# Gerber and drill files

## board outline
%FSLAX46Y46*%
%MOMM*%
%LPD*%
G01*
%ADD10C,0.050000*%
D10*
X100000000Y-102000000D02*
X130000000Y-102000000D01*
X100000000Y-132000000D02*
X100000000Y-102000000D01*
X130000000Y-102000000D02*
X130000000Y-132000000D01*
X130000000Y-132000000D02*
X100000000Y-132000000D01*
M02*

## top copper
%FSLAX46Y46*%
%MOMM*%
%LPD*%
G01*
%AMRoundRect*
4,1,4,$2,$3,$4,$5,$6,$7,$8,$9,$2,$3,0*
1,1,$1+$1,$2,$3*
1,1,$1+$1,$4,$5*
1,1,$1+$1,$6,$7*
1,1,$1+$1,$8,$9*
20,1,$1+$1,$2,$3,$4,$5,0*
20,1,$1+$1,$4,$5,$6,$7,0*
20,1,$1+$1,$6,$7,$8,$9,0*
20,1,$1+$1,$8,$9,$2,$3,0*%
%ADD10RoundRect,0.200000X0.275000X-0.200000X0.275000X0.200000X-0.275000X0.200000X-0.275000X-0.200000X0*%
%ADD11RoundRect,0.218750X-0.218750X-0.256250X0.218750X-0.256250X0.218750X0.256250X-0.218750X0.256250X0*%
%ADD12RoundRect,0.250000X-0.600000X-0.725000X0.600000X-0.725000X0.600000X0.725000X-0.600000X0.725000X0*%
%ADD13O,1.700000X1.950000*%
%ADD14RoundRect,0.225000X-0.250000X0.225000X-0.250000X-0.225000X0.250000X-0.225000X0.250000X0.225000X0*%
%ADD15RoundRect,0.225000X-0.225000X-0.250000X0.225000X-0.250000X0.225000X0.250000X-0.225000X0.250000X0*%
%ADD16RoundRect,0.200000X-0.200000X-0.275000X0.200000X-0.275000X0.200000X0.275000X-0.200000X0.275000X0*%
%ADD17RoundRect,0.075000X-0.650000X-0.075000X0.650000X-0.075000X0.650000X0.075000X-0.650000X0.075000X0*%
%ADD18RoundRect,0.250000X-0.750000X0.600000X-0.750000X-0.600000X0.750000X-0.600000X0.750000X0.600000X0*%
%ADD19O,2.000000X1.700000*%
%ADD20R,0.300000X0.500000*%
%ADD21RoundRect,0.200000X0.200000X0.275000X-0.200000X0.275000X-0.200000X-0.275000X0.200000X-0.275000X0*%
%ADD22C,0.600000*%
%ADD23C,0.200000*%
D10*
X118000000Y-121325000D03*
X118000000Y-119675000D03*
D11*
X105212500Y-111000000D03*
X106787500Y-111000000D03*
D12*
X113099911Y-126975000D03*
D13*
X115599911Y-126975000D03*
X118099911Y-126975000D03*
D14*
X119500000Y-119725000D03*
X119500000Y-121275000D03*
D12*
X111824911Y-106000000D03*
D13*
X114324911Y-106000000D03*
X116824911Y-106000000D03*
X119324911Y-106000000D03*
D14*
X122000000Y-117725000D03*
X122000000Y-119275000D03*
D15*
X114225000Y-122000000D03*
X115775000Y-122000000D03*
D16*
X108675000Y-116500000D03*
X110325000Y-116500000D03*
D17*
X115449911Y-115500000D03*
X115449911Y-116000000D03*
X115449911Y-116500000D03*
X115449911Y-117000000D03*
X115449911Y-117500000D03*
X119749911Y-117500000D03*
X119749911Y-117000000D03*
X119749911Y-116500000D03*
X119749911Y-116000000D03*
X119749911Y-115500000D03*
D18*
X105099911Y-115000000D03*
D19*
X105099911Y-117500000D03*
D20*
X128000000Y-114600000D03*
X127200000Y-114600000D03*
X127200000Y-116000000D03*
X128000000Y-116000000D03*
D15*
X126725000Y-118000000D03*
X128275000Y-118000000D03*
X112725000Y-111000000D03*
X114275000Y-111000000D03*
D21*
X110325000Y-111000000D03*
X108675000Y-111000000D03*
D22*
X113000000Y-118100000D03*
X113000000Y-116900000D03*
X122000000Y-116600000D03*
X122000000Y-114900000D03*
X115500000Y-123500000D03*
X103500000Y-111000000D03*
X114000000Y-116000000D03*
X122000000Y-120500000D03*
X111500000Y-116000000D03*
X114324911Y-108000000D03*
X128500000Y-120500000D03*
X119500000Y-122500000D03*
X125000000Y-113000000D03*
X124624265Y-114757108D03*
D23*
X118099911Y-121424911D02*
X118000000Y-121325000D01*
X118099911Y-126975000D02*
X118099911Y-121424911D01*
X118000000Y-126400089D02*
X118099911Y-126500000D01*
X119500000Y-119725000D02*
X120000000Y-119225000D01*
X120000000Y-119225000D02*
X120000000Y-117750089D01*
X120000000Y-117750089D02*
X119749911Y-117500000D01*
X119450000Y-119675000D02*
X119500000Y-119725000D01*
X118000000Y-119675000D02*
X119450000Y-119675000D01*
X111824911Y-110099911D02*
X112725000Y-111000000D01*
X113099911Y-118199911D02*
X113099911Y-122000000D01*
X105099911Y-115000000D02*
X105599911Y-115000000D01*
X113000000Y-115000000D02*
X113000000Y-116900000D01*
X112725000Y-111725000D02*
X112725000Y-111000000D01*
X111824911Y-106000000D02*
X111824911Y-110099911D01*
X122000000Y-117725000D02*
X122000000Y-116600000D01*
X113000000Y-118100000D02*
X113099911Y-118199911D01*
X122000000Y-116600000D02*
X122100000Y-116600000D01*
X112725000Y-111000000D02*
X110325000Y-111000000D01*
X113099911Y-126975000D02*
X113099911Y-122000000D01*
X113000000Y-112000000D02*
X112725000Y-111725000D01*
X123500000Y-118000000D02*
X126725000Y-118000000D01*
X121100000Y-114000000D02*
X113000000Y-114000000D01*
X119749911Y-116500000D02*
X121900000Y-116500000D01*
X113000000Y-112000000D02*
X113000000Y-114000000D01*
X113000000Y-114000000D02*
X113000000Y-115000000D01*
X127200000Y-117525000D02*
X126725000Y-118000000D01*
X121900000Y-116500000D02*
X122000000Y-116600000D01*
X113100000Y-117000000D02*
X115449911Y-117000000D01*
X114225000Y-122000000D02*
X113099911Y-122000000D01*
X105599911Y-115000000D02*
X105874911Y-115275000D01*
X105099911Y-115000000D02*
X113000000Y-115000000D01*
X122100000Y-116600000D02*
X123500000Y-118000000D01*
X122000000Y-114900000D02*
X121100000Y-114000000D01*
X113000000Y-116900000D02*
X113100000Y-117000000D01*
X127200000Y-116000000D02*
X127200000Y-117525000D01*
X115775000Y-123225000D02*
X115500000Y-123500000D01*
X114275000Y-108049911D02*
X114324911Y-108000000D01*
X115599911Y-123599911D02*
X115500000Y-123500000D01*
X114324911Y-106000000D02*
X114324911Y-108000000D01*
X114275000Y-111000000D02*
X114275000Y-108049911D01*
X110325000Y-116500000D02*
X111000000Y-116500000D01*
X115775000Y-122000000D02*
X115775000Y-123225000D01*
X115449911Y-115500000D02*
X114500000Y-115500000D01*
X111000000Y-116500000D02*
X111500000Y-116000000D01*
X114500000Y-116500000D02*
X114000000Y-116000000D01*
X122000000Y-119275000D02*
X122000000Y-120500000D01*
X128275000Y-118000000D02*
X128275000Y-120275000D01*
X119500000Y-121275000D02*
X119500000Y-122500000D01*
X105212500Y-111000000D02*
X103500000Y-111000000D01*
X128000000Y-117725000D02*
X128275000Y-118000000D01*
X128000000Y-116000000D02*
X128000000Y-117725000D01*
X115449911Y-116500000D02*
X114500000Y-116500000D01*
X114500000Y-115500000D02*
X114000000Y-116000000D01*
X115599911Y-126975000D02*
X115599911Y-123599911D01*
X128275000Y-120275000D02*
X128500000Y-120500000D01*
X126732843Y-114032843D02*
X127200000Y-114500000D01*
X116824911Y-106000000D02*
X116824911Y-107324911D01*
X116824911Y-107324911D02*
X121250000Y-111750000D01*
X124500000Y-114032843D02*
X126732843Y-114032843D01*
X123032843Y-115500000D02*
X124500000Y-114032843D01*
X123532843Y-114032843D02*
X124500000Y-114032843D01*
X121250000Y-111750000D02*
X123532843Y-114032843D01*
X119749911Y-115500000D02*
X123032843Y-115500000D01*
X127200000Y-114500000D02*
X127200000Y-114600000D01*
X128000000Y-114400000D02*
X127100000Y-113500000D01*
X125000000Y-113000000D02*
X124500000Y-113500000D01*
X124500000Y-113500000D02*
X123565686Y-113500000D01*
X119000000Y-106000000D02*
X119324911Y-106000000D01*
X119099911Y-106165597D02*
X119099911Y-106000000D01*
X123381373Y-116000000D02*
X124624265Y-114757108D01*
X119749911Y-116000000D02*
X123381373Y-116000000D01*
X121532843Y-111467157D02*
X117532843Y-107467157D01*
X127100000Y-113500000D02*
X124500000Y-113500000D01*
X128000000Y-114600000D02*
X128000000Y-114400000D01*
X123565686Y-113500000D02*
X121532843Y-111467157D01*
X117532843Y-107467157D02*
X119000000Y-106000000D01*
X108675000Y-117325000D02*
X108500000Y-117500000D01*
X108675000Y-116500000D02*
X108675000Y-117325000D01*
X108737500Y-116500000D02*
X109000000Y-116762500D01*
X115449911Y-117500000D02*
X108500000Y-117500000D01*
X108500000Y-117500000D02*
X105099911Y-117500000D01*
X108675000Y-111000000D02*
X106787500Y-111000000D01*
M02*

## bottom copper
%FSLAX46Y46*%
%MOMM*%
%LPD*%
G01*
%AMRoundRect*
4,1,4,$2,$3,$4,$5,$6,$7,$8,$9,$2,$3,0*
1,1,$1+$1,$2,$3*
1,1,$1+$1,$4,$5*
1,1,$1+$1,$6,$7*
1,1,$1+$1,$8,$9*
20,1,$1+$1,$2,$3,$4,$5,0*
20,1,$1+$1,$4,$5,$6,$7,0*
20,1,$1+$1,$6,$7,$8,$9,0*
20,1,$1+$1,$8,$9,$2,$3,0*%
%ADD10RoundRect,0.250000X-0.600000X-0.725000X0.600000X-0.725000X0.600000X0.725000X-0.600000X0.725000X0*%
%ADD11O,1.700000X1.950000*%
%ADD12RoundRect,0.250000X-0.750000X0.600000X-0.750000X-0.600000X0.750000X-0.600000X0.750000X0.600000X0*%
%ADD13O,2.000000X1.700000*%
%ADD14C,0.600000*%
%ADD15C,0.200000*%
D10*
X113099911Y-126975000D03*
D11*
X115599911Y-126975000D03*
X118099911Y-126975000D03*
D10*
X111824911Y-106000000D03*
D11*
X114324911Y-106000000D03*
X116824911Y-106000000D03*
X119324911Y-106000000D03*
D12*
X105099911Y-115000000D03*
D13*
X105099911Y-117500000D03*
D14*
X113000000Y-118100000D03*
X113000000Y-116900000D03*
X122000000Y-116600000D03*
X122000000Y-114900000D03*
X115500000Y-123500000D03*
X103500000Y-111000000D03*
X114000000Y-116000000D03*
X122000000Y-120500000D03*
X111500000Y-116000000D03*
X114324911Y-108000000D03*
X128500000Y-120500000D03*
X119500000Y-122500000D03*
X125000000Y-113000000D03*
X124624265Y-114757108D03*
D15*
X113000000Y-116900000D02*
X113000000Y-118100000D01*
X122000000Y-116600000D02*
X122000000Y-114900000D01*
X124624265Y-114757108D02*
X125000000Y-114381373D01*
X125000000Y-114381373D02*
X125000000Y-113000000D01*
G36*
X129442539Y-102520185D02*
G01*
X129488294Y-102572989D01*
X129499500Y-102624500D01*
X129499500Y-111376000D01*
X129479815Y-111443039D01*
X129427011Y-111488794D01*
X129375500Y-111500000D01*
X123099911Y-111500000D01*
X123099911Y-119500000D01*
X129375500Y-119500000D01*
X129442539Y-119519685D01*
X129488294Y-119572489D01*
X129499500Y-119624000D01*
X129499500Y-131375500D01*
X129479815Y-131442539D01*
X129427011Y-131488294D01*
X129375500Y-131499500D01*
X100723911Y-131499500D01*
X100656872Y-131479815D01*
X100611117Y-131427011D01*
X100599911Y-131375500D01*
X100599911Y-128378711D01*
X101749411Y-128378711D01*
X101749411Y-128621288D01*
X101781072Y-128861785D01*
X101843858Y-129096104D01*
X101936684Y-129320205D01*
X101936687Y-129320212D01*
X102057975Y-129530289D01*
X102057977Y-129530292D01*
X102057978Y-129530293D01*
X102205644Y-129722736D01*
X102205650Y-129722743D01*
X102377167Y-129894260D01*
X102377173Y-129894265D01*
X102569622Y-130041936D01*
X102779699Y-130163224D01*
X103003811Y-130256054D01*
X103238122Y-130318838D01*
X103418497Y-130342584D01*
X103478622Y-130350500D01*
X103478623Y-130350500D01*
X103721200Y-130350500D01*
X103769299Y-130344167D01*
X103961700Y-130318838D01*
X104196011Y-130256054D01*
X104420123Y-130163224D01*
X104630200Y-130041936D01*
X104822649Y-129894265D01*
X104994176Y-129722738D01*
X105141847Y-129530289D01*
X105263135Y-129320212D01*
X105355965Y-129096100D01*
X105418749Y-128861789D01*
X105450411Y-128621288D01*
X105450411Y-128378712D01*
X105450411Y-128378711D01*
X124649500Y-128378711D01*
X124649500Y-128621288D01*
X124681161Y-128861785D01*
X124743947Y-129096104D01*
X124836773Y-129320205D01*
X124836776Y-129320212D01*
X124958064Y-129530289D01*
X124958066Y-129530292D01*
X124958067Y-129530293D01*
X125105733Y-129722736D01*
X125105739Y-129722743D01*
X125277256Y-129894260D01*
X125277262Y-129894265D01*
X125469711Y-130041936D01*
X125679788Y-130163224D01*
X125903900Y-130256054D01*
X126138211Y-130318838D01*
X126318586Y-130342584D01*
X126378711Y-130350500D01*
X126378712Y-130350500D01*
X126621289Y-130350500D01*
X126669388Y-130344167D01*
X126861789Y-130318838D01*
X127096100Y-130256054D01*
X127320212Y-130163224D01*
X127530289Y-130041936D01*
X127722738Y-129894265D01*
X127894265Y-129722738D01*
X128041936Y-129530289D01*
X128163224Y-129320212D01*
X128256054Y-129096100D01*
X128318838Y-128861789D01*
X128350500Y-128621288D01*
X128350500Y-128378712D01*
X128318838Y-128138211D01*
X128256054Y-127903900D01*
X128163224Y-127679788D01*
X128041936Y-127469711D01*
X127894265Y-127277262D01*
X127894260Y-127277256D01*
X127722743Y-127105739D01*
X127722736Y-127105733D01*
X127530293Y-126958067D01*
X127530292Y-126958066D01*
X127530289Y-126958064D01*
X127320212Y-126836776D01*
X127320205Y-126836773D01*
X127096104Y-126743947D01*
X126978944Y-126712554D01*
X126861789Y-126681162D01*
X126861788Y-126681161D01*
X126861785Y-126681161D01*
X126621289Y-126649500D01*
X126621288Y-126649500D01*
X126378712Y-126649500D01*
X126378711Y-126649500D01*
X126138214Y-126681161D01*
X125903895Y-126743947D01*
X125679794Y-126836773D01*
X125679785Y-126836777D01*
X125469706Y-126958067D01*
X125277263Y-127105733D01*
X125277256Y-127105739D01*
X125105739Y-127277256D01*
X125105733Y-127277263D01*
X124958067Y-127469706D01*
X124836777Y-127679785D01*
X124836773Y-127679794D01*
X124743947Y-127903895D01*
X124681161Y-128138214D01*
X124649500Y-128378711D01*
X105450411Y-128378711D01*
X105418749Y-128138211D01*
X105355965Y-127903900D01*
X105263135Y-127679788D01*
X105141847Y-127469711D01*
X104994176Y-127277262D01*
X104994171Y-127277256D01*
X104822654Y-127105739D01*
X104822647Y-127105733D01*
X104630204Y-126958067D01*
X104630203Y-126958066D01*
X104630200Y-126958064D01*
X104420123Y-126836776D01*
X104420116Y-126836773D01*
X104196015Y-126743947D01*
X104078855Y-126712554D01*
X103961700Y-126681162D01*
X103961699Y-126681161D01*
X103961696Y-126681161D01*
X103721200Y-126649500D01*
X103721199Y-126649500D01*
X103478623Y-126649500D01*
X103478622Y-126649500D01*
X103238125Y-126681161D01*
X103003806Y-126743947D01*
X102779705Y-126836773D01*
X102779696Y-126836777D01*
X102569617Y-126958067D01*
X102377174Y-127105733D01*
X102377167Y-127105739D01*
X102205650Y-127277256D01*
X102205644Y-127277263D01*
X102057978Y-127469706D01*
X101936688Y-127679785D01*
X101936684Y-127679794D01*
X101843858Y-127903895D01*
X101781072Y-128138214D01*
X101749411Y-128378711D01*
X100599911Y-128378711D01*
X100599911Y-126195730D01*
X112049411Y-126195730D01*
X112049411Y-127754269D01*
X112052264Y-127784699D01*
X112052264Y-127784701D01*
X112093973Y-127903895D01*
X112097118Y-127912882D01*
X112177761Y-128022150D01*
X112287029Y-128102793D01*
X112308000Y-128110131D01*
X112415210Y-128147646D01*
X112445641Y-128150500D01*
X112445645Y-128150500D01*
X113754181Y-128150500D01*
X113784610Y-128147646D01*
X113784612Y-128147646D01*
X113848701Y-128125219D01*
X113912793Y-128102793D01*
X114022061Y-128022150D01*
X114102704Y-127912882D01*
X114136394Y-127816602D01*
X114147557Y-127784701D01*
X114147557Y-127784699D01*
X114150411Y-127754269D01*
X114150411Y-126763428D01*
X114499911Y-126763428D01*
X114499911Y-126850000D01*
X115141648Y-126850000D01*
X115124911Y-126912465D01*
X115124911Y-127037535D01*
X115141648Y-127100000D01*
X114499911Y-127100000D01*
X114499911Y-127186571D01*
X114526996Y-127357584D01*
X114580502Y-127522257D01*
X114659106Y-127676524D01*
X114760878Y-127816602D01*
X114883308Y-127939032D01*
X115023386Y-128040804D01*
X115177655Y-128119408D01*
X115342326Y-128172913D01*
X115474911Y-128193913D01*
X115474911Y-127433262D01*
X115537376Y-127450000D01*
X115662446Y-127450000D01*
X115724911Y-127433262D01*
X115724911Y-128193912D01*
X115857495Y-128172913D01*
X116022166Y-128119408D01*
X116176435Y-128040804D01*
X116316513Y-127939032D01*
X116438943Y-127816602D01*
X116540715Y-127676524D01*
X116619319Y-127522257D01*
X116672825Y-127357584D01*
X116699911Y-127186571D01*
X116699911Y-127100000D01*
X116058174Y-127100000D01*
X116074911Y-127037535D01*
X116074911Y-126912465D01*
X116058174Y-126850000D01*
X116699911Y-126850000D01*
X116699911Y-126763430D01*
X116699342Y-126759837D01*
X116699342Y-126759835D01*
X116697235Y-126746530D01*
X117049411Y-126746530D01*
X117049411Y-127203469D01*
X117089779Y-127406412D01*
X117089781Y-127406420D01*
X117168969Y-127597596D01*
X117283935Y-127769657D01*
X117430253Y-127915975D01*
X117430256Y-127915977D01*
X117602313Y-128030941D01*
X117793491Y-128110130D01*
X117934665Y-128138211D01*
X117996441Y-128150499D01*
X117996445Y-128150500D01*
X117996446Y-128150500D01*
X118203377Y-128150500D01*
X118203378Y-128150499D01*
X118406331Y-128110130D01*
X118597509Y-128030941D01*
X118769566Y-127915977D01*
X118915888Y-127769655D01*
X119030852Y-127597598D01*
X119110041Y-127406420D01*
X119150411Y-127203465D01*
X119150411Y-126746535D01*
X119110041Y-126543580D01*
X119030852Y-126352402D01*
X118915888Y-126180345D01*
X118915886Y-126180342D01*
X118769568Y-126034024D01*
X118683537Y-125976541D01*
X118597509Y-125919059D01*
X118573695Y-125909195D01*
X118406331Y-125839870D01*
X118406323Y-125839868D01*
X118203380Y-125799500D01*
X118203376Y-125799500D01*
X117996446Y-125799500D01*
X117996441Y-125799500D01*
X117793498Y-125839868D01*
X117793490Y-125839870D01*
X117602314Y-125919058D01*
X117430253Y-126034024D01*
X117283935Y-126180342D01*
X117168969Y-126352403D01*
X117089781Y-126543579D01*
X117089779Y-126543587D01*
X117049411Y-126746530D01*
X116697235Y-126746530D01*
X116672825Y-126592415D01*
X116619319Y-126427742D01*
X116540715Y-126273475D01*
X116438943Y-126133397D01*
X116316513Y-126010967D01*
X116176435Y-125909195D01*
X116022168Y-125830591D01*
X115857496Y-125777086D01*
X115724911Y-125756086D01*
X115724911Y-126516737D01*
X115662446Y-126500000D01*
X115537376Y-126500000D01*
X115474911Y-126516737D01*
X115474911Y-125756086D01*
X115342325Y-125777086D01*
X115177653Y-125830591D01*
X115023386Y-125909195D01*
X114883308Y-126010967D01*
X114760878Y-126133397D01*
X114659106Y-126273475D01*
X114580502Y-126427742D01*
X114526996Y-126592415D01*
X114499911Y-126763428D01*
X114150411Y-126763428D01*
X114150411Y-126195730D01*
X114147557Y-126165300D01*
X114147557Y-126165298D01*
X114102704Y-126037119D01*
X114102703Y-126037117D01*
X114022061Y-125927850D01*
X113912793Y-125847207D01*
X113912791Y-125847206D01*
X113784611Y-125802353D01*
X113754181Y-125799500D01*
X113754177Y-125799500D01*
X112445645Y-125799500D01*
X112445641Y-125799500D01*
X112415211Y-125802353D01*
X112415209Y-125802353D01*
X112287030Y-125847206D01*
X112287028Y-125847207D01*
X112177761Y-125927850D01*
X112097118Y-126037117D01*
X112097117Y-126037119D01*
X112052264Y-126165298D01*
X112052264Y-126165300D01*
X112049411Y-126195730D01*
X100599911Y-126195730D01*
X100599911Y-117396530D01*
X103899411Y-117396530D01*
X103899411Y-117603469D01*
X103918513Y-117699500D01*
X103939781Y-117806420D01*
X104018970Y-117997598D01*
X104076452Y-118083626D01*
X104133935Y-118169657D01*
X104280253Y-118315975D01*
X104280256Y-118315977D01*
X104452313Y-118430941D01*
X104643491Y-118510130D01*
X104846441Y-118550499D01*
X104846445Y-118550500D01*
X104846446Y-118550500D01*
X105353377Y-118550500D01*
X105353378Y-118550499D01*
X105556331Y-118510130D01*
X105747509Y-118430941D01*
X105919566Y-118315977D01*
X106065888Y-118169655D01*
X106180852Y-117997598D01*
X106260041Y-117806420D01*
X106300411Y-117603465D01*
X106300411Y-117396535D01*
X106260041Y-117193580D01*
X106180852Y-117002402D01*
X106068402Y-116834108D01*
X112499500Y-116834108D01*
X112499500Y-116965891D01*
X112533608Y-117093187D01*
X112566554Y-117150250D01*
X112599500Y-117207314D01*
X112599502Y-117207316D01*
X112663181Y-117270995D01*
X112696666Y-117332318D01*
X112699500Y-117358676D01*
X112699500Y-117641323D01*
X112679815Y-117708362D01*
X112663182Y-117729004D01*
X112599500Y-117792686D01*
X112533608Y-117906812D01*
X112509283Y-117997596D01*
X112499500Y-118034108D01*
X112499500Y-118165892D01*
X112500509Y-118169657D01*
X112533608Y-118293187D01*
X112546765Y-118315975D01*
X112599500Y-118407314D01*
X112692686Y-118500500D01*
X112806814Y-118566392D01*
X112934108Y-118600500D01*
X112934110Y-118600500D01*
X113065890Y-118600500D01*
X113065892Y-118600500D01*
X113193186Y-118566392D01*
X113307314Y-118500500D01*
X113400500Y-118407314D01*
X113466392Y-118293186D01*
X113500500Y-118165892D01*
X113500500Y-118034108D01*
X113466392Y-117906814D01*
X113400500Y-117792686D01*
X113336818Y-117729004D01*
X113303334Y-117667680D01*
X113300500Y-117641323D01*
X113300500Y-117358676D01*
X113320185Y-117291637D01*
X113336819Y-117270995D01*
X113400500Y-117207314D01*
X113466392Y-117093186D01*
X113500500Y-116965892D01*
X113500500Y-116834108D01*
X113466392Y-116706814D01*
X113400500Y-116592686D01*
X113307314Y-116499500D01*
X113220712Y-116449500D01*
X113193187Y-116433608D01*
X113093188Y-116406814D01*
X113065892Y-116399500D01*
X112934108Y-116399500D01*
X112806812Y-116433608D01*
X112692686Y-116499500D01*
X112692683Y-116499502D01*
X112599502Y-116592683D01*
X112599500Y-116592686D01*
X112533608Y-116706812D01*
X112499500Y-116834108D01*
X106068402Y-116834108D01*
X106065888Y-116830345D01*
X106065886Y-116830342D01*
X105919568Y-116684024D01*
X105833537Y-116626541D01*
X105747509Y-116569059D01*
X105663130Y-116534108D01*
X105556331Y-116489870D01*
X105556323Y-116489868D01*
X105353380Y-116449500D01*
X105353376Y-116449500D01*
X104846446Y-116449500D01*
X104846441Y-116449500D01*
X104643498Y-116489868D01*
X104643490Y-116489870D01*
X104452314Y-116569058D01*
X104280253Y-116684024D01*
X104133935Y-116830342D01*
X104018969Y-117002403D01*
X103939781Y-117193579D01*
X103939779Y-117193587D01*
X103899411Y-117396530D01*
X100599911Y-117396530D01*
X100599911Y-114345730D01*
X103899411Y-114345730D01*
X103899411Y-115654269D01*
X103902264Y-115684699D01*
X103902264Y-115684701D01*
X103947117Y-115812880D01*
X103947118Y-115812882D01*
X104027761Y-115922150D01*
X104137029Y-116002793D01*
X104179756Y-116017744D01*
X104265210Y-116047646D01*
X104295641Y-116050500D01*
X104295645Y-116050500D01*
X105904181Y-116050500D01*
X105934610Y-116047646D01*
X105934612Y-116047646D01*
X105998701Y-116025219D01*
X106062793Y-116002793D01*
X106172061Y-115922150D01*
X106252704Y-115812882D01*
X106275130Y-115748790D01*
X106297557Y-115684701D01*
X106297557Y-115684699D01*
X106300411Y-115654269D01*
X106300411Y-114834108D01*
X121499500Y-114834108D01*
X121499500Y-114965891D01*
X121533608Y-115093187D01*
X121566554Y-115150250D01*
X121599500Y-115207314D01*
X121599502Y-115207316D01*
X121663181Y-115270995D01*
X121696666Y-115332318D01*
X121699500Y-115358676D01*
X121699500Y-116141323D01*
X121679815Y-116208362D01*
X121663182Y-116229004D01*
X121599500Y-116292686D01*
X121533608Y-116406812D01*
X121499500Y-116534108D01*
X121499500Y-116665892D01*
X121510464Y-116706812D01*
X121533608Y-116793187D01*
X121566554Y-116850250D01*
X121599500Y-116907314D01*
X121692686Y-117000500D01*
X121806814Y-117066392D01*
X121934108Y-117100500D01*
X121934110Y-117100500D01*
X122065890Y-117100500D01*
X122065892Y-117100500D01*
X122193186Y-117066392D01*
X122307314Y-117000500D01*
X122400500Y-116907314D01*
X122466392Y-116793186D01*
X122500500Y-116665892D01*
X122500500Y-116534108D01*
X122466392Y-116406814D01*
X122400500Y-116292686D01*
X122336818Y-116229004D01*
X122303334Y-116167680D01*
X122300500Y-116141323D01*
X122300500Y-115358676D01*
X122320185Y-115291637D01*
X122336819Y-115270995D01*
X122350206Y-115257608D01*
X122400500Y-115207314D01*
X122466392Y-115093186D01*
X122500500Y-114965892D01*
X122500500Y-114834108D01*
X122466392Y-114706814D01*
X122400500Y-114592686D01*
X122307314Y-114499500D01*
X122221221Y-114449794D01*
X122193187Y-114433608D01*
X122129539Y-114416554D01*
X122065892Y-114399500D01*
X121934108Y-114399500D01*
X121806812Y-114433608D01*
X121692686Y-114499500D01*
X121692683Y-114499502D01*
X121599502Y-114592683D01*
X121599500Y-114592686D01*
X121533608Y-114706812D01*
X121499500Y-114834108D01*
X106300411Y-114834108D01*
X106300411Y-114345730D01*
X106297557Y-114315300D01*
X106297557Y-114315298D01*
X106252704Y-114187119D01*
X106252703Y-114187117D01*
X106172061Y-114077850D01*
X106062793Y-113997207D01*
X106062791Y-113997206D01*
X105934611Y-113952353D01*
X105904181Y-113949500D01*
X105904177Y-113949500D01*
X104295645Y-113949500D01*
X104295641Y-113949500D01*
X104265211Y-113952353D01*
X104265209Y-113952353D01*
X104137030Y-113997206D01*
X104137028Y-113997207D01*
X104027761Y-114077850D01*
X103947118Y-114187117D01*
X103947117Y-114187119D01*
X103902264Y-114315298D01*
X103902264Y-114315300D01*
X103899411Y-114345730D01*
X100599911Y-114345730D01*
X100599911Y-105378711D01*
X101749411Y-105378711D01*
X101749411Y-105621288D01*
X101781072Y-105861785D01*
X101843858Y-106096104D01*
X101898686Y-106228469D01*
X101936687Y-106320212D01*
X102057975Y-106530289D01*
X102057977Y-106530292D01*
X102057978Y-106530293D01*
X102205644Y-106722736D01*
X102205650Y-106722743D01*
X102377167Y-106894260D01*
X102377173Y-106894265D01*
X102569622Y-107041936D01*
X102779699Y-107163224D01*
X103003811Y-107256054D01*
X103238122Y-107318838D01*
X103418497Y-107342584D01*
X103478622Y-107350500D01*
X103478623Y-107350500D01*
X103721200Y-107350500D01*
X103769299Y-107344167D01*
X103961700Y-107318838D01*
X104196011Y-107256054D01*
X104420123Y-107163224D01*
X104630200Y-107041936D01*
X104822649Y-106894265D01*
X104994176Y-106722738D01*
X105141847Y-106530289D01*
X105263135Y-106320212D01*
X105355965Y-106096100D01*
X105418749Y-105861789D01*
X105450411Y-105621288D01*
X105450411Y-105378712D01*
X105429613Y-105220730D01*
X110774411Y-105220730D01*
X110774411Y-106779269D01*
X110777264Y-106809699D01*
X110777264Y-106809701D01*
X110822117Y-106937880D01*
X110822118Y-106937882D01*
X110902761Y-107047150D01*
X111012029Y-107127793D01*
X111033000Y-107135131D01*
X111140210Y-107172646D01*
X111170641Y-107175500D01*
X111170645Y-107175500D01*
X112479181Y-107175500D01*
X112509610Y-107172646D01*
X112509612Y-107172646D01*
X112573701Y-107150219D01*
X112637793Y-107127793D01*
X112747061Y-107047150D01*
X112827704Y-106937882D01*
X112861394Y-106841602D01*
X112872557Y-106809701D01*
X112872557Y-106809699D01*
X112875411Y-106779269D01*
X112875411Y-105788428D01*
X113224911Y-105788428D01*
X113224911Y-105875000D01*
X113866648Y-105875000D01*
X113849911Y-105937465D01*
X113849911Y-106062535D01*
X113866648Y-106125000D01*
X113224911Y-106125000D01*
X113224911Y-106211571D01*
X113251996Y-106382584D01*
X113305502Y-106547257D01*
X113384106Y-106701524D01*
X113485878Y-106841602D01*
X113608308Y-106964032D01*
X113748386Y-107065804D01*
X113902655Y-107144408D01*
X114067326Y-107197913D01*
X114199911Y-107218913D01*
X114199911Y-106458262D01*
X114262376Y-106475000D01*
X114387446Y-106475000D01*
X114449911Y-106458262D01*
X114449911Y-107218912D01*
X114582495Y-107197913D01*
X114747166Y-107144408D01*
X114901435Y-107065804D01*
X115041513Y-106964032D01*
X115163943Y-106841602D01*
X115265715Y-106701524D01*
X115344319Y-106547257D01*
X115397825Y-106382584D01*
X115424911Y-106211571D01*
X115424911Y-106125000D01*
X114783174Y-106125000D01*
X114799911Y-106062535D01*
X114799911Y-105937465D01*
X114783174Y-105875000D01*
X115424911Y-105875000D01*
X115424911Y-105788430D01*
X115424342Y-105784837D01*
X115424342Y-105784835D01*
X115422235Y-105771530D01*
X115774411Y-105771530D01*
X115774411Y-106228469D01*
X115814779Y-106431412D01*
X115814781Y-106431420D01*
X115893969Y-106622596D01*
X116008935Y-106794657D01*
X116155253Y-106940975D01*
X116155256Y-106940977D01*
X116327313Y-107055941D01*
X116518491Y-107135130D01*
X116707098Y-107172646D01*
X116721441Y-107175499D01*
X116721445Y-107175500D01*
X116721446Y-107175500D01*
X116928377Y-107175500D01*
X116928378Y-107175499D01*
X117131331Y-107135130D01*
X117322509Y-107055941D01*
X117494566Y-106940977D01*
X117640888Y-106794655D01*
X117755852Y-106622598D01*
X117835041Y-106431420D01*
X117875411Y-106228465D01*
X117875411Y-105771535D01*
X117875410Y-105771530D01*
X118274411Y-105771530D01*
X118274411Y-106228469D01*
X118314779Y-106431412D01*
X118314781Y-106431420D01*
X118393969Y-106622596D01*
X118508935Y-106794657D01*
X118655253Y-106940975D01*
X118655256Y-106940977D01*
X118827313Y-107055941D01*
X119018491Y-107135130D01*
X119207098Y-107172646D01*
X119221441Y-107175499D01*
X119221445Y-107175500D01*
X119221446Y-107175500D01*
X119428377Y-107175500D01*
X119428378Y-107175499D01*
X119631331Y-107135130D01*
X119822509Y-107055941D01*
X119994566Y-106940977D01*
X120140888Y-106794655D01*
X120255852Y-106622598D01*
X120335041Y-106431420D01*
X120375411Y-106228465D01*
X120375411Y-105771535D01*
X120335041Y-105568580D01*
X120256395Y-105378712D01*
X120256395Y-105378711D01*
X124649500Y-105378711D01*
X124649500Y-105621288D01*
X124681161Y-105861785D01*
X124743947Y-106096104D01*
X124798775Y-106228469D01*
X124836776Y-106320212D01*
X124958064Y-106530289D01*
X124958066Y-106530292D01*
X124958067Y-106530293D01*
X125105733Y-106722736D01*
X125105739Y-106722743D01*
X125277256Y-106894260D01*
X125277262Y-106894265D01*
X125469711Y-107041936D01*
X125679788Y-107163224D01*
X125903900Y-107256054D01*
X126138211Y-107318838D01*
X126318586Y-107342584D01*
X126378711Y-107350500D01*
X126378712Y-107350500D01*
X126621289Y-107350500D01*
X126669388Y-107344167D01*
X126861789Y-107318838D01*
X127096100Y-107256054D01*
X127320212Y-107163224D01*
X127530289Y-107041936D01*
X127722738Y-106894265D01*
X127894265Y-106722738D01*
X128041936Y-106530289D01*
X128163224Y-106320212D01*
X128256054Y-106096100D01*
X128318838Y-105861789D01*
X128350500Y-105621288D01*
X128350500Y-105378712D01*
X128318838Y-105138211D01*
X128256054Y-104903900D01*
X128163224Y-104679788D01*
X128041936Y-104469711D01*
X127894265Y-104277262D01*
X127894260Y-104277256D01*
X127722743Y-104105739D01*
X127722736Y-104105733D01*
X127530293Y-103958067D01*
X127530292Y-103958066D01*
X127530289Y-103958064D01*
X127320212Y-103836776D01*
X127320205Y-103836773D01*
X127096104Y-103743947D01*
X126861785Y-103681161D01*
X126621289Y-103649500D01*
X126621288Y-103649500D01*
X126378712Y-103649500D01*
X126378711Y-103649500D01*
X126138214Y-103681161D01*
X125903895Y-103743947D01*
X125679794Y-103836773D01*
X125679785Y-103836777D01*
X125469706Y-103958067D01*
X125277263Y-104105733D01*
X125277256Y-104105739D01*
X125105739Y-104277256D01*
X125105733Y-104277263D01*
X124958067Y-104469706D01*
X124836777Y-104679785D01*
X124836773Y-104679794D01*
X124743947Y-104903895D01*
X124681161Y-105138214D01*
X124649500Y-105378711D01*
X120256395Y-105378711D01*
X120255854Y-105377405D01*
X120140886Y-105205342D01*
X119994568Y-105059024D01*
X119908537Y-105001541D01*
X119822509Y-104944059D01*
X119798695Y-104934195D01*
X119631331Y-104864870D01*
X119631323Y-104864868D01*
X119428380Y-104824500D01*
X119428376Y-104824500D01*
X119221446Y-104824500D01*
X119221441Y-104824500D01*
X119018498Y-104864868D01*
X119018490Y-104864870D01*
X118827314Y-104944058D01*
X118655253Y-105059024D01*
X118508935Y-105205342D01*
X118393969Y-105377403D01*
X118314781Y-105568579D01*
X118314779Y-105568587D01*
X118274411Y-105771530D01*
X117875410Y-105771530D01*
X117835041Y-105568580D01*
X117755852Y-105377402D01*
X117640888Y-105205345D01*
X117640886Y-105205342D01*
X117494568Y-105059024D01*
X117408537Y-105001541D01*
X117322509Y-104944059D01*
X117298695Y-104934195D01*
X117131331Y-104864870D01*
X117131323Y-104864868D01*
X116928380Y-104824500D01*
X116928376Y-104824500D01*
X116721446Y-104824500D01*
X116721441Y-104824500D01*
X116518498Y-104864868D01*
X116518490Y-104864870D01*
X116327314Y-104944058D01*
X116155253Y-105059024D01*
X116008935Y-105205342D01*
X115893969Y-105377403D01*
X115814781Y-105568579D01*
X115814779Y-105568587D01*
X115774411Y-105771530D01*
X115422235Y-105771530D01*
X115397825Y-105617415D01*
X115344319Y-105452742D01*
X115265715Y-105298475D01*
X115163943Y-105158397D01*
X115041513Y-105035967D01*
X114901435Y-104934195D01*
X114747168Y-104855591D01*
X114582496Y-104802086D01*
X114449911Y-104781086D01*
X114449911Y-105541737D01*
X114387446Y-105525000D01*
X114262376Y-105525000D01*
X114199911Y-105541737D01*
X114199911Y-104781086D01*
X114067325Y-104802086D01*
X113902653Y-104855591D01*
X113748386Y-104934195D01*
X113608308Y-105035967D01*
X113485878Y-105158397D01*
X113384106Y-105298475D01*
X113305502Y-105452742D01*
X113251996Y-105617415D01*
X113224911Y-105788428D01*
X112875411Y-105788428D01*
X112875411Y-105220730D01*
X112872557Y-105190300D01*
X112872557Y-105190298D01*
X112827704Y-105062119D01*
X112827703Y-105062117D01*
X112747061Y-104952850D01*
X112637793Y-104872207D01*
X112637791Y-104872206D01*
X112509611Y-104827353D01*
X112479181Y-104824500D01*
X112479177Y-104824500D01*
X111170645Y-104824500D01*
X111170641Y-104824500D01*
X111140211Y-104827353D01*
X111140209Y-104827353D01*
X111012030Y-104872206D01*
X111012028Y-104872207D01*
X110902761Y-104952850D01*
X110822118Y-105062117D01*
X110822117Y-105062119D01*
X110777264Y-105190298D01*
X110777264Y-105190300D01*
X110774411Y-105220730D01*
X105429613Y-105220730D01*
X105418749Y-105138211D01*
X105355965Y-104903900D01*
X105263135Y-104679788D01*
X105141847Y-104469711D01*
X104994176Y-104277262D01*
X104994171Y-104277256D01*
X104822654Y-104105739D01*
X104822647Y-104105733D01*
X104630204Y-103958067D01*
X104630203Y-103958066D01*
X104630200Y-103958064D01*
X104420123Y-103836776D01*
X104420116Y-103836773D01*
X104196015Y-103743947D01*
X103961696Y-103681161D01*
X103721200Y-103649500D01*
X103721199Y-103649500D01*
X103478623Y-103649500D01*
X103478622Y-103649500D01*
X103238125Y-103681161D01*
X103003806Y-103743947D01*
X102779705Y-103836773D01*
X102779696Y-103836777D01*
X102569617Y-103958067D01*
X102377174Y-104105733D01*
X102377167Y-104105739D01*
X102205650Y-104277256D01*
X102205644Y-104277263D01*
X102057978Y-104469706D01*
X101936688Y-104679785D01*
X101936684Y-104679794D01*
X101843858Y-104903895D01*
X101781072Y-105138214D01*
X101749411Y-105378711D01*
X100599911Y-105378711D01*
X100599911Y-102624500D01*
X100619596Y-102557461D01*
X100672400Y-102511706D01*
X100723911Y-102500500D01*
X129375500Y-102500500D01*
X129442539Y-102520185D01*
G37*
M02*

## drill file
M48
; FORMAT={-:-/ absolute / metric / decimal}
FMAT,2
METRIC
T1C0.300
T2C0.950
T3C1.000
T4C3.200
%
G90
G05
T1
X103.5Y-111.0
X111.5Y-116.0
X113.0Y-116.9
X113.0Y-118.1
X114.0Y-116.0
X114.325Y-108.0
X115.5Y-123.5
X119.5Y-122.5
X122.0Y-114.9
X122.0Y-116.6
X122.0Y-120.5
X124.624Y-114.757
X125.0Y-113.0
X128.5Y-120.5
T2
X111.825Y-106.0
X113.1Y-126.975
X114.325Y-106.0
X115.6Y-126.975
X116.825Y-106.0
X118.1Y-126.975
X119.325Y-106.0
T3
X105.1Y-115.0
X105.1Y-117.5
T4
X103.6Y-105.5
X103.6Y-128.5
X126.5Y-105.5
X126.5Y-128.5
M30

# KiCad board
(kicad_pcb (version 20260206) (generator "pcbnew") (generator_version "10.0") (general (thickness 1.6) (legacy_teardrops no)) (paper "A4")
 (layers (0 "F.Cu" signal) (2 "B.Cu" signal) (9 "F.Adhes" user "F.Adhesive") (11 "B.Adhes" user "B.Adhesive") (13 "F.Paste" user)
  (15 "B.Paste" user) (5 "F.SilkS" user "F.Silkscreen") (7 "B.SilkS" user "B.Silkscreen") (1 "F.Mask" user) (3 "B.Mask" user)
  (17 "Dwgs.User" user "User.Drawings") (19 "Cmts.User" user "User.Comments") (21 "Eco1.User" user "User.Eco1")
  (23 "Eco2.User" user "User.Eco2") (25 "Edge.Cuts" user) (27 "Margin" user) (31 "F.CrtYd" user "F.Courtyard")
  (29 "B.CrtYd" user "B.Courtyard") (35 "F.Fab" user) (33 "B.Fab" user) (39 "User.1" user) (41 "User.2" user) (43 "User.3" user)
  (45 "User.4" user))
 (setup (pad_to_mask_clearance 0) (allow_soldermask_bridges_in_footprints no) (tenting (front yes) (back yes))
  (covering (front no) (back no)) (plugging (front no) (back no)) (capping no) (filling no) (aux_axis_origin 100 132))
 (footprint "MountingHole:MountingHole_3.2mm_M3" (layer "F.Cu") (at 126.5 105.5)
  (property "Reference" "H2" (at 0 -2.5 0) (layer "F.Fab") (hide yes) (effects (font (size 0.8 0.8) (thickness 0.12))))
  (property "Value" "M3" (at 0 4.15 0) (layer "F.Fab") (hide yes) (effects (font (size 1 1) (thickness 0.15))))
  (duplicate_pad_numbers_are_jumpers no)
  (pad "" np_thru_hole circle (at 0 0) (size 3.2 3.2) (drill 3.2) (layers "*.Cu" "*.Mask")))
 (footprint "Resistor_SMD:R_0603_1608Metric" (layer "F.Cu") (at 118 120.5 90)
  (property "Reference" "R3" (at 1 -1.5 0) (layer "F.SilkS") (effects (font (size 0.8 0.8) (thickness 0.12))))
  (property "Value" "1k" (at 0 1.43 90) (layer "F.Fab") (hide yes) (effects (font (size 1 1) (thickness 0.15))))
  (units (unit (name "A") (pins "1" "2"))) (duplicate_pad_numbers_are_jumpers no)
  (pad "1" smd roundrect (at -0.825 0 90) (size 0.8 0.95) (layers "F.Cu" "F.Mask" "F.Paste") (roundrect_rratio 0.25) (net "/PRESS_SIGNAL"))
  (pad "2" smd roundrect (at 0.825 0 90) (size 0.8 0.95) (layers "F.Cu" "F.Mask" "F.Paste") (roundrect_rratio 0.25) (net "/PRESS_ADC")))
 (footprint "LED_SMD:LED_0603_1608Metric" (layer "F.Cu") (at 106 111)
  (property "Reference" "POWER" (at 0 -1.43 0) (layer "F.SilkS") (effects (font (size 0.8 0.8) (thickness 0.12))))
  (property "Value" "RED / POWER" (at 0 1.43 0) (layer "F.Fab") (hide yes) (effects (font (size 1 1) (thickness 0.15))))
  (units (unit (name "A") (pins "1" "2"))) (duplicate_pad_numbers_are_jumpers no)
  (pad "1" smd roundrect (at -0.7875 0) (size 0.875 0.95) (layers "F.Cu" "F.Mask" "F.Paste") (roundrect_rratio 0.25) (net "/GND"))
  (pad "2" smd roundrect (at 0.7875 0) (size 0.875 0.95) (layers "F.Cu" "F.Mask" "F.Paste") (roundrect_rratio 0.25) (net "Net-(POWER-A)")))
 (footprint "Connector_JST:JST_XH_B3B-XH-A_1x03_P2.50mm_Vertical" (layer "F.Cu") (at 113.099911 126.975)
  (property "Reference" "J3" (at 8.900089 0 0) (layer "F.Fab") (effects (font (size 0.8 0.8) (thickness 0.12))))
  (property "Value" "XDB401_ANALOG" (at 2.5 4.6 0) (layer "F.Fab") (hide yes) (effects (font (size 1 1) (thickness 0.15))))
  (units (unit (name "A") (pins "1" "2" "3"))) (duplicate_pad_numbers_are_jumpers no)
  (pad "1" thru_hole roundrect (at 0 0) (size 1.7 1.95) (drill 0.95) (layers "*.Cu" "*.Mask") (remove_unused_layers no)
   (roundrect_rratio 0.147059) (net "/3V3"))
  (pad "2" thru_hole oval (at 2.5 0) (size 1.7 1.95) (drill 0.95) (layers "*.Cu" "*.Mask") (remove_unused_layers no) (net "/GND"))
  (pad "3" thru_hole oval (at 5 0) (size 1.7 1.95) (drill 0.95) (layers "*.Cu" "*.Mask") (remove_unused_layers no) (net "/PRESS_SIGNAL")))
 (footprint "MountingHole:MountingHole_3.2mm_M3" (layer "F.Cu") (at 126.5 128.5)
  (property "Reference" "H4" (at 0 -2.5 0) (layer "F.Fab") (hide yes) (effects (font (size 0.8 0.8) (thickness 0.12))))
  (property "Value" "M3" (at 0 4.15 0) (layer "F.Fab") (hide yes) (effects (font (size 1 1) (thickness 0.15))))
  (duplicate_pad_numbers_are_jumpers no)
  (pad "" np_thru_hole circle (at 0 0) (size 3.2 3.2) (drill 3.2) (layers "*.Cu" "*.Mask")))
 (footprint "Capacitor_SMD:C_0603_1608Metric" (layer "F.Cu") (at 119.5 120.5 -90)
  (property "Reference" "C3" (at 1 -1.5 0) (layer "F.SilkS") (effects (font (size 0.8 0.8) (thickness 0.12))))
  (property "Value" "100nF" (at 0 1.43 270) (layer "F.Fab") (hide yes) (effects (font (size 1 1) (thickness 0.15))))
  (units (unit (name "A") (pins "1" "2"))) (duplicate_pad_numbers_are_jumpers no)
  (pad "1" smd roundrect (at -0.775 0 270) (size 0.9 0.95) (layers "F.Cu" "F.Mask" "F.Paste") (roundrect_rratio 0.25) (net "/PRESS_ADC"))
  (pad "2" smd roundrect (at 0.775 0 270) (size 0.9 0.95) (layers "F.Cu" "F.Mask" "F.Paste") (roundrect_rratio 0.25) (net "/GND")))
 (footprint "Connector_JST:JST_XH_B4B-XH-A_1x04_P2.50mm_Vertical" (layer "F.Cu") (at 111.824911 106)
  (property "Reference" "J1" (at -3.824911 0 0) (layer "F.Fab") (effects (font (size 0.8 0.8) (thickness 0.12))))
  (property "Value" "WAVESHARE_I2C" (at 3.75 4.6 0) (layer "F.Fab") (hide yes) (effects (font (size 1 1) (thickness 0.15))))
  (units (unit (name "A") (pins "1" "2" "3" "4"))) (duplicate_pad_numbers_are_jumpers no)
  (pad "1" thru_hole roundrect (at 0 0) (size 1.7 1.95) (drill 0.95) (layers "*.Cu" "*.Mask") (remove_unused_layers no)
   (roundrect_rratio 0.147059) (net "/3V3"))
  (pad "2" thru_hole oval (at 2.5 0) (size 1.7 1.95) (drill 0.95) (layers "*.Cu" "*.Mask") (remove_unused_layers no) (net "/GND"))
  (pad "3" thru_hole oval (at 5 0) (size 1.7 1.95) (drill 0.95) (layers "*.Cu" "*.Mask") (remove_unused_layers no) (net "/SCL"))
  (pad "4" thru_hole oval (at 7.5 0) (size 1.7 1.95) (drill 0.95) (layers "*.Cu" "*.Mask") (remove_unused_layers no) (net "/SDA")))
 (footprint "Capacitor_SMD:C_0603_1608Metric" (layer "F.Cu") (at 122 118.5 -90)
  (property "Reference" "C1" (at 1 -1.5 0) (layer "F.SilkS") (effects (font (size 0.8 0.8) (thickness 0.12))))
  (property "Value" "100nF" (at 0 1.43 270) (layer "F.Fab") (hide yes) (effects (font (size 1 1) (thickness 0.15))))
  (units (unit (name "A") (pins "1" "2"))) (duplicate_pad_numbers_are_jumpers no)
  (pad "1" smd roundrect (at -0.775 0 270) (size 0.9 0.95) (layers "F.Cu" "F.Mask" "F.Paste") (roundrect_rratio 0.25) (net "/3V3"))
  (pad "2" smd roundrect (at 0.775 0 270) (size 0.9 0.95) (layers "F.Cu" "F.Mask" "F.Paste") (roundrect_rratio 0.25) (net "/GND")))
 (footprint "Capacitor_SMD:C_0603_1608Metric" (layer "F.Cu") (at 115 122)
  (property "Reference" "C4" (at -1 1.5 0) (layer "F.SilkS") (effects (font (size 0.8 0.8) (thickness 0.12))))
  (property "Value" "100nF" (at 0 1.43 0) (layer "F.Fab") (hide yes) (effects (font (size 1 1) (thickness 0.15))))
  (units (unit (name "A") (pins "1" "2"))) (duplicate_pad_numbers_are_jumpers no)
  (pad "1" smd roundrect (at -0.775 0) (size 0.9 0.95) (layers "F.Cu" "F.Mask" "F.Paste") (roundrect_rratio 0.25) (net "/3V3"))
  (pad "2" smd roundrect (at 0.775 0) (size 0.9 0.95) (layers "F.Cu" "F.Mask" "F.Paste") (roundrect_rratio 0.25) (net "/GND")))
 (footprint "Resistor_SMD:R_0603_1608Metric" (layer "F.Cu") (at 109.5 116.5)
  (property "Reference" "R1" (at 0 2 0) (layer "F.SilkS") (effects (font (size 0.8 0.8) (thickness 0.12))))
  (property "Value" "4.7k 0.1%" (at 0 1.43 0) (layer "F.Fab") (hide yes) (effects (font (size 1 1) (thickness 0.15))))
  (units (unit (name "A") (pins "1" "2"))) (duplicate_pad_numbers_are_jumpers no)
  (pad "1" smd roundrect (at -0.825 0) (size 0.8 0.95) (layers "F.Cu" "F.Mask" "F.Paste") (roundrect_rratio 0.25) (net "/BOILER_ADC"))
  (pad "2" smd roundrect (at 0.825 0) (size 0.8 0.95) (layers "F.Cu" "F.Mask" "F.Paste") (roundrect_rratio 0.25) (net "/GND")))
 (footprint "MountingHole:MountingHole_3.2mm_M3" (layer "F.Cu") (at 103.599911 128.5)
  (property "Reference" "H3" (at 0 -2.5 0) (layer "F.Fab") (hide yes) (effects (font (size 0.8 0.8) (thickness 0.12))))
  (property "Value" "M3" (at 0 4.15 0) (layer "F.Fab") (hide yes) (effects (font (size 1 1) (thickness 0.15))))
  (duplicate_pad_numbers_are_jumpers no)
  (pad "" np_thru_hole circle (at 0 0) (size 3.2 3.2) (drill 3.2) (layers "*.Cu" "*.Mask")))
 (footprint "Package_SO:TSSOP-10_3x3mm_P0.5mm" (layer "F.Cu") (at 117.599911 116.5)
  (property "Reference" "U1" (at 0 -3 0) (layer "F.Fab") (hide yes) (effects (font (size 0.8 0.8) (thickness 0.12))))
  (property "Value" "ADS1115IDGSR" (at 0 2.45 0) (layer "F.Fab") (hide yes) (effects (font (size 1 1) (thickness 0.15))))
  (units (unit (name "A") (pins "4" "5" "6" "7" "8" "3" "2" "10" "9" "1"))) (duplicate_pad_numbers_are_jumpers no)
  (pad "1" smd roundrect (at -2.15 -1) (size 1.45 0.3) (layers "F.Cu" "F.Mask" "F.Paste") (roundrect_rratio 0.25) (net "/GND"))
  (pad "2" smd roundrect (at -2.15 -0.5) (size 1.45 0.3) (layers "F.Cu" "F.Mask" "F.Paste") (roundrect_rratio 0.25)
   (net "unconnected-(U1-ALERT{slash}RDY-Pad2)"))
  (pad "3" smd roundrect (at -2.15 0) (size 1.45 0.3) (layers "F.Cu" "F.Mask" "F.Paste") (roundrect_rratio 0.25) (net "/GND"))
  (pad "4" smd roundrect (at -2.15 0.5) (size 1.45 0.3) (layers "F.Cu" "F.Mask" "F.Paste") (roundrect_rratio 0.25) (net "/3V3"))
  (pad "5" smd roundrect (at -2.15 1) (size 1.45 0.3) (layers "F.Cu" "F.Mask" "F.Paste") (roundrect_rratio 0.25) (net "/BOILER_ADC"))
  (pad "6" smd roundrect (at 2.15 1) (size 1.45 0.3) (layers "F.Cu" "F.Mask" "F.Paste") (roundrect_rratio 0.25) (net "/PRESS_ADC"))
  (pad "7" smd roundrect (at 2.15 0.5) (size 1.45 0.3) (layers "F.Cu" "F.Mask" "F.Paste") (roundrect_rratio 0.25)
   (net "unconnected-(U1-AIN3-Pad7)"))
  (pad "8" smd roundrect (at 2.15 0) (size 1.45 0.3) (layers "F.Cu" "F.Mask" "F.Paste") (roundrect_rratio 0.25) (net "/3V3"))
  (pad "9" smd roundrect (at 2.15 -0.5) (size 1.45 0.3) (layers "F.Cu" "F.Mask" "F.Paste") (roundrect_rratio 0.25) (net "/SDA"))
  (pad "10" smd roundrect (at 2.15 -1) (size 1.45 0.3) (layers "F.Cu" "F.Mask" "F.Paste") (roundrect_rratio 0.25) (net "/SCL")))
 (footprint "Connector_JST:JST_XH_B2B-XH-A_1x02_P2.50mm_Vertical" (layer "F.Cu") (at 105.099911 115 -90)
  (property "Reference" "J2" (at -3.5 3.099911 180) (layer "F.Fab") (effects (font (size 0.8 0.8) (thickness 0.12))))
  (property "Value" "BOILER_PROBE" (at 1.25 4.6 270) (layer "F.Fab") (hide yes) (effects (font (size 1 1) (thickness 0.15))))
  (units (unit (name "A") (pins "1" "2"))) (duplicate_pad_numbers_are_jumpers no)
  (pad "1" thru_hole roundrect (at 0 0 270) (size 1.7 2) (drill 1) (layers "*.Cu" "*.Mask") (remove_unused_layers no)
   (roundrect_rratio 0.147059) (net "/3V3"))
  (pad "2" thru_hole oval (at 2.5 0 270) (size 1.7 2) (drill 1) (layers "*.Cu" "*.Mask") (remove_unused_layers no) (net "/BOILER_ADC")))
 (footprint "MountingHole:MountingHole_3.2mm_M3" (layer "F.Cu") (at 103.599911 105.5)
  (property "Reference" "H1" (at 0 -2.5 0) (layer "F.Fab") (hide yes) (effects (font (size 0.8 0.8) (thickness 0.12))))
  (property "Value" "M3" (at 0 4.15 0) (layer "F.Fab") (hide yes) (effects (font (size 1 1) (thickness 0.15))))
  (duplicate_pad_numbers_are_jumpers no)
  (pad "" np_thru_hole circle (at 0 0) (size 3.2 3.2) (drill 3.2) (layers "*.Cu" "*.Mask")))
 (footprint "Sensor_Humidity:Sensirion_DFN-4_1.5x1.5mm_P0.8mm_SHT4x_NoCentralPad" (layer "F.Cu") (at 127.6 115.3 -90)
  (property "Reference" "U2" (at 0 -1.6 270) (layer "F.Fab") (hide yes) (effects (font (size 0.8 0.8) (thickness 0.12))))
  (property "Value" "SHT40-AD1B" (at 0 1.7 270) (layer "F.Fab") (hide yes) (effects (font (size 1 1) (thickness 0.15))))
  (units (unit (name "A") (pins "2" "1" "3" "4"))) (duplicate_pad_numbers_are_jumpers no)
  (pad "1" smd rect (at -0.7 -0.4 270) (size 0.5 0.3) (layers "F.Cu" "F.Mask" "F.Paste") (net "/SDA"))
  (pad "2" smd rect (at -0.7 0.4 270) (size 0.5 0.3) (layers "F.Cu" "F.Mask" "F.Paste") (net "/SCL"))
  (pad "3" smd rect (at 0.7 0.4 270) (size 0.5 0.3) (layers "F.Cu" "F.Mask" "F.Paste") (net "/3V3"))
  (pad "4" smd rect (at 0.7 -0.4 270) (size 0.5 0.3) (layers "F.Cu" "F.Mask" "F.Paste") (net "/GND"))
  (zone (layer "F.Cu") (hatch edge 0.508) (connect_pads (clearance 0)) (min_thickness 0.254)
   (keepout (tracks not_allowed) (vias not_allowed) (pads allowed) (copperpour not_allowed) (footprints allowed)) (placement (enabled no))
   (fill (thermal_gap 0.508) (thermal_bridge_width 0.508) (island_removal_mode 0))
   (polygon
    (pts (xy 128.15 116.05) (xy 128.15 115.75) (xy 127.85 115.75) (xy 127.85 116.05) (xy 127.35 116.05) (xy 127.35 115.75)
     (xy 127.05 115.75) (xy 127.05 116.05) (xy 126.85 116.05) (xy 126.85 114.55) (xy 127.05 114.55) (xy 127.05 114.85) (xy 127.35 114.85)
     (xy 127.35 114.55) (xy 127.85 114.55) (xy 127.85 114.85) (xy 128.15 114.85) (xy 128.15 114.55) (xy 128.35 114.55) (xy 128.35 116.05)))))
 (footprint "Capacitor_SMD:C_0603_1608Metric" (layer "F.Cu") (at 127.5 118)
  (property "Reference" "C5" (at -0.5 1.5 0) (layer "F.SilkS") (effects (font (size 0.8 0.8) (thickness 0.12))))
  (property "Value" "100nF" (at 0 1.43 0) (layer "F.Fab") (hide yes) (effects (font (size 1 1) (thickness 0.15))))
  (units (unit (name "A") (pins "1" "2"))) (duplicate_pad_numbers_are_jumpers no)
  (pad "1" smd roundrect (at -0.775 0) (size 0.9 0.95) (layers "F.Cu" "F.Mask" "F.Paste") (roundrect_rratio 0.25) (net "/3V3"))
  (pad "2" smd roundrect (at 0.775 0) (size 0.9 0.95) (layers "F.Cu" "F.Mask" "F.Paste") (roundrect_rratio 0.25) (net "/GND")))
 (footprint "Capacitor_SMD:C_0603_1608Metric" (layer "F.Cu") (at 113.5 111)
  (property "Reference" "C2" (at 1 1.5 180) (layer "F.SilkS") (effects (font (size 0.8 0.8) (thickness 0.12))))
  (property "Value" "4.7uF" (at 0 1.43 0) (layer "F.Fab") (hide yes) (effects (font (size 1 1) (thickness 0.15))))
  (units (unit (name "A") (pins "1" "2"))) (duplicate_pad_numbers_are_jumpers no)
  (pad "1" smd roundrect (at -0.775 0) (size 0.9 0.95) (layers "F.Cu" "F.Mask" "F.Paste") (roundrect_rratio 0.25) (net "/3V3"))
  (pad "2" smd roundrect (at 0.775 0) (size 0.9 0.95) (layers "F.Cu" "F.Mask" "F.Paste") (roundrect_rratio 0.25) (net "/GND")))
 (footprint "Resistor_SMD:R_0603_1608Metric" (layer "F.Cu") (at 109.5 111 180)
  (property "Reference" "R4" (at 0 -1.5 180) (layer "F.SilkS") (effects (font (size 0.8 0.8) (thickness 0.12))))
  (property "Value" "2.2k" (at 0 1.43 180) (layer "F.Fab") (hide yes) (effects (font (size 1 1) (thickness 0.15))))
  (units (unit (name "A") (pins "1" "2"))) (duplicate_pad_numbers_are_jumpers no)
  (pad "1" smd roundrect (at -0.825 0 180) (size 0.8 0.95) (layers "F.Cu" "F.Mask" "F.Paste") (roundrect_rratio 0.25) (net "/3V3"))
  (pad "2" smd roundrect (at 0.825 0 180) (size 0.8 0.95) (layers "F.Cu" "F.Mask" "F.Paste") (roundrect_rratio 0.25) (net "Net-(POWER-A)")))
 (gr_line (start 100 102) (end 130 102) (stroke (width 0.05) (type default)) (layer "Edge.Cuts"))
 (gr_line (start 100 132) (end 100 102) (stroke (width 0.05) (type default)) (layer "Edge.Cuts"))
 (gr_line (start 130 102) (end 130 132) (stroke (width 0.05) (type default)) (layer "Edge.Cuts"))
 (gr_line (start 130 132) (end 100 132) (stroke (width 0.05) (type default)) (layer "Edge.Cuts"))
 (segment (start 118.099911 121.424911) (end 118 121.325) (width 0.2) (layer "F.Cu") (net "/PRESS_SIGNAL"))
 (segment (start 118.099911 126.975) (end 118.099911 121.424911) (width 0.2) (layer "F.Cu") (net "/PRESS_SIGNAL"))
 (segment (start 118 126.400089) (end 118.099911 126.5) (width 0.2) (layer "F.Cu") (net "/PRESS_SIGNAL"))
 (segment (start 119.5 119.725) (end 120 119.225) (width 0.2) (layer "F.Cu") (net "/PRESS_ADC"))
 (segment (start 120 119.225) (end 120 117.750089) (width 0.2) (layer "F.Cu") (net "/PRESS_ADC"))
 (segment (start 120 117.750089) (end 119.749911 117.5) (width 0.2) (layer "F.Cu") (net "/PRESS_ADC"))
 (segment (start 119.45 119.675) (end 119.5 119.725) (width 0.2) (layer "F.Cu") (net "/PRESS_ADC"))
 (segment (start 118 119.675) (end 119.45 119.675) (width 0.2) (layer "F.Cu") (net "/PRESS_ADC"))
 (segment (start 111.824911 110.099911) (end 112.725 111) (width 0.2) (layer "F.Cu") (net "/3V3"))
 (segment (start 113.099911 118.199911) (end 113.099911 122) (width 0.2) (layer "F.Cu") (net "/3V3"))
 (segment (start 105.099911 115) (end 105.599911 115) (width 0.2) (layer "F.Cu") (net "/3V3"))
 (segment (start 113 115) (end 113 116.9) (width 0.2) (layer "F.Cu") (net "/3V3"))
 (segment (start 112.725 111.725) (end 112.725 111) (width 0.2) (layer "F.Cu") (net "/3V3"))
 (segment (start 111.824911 106) (end 111.824911 110.099911) (width 0.2) (layer "F.Cu") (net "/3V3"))
 (segment (start 122 117.725) (end 122 116.6) (width 0.2) (layer "F.Cu") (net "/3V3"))
 (segment (start 113 118.1) (end 113.099911 118.199911) (width 0.2) (layer "F.Cu") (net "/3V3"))
 (segment (start 122 116.6) (end 122.1 116.6) (width 0.2) (layer "F.Cu") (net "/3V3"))
 (segment (start 112.725 111) (end 110.325 111) (width 0.2) (layer "F.Cu") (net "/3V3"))
 (segment (start 113.099911 126.975) (end 113.099911 122) (width 0.2) (layer "F.Cu") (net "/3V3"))
 (segment (start 113 112) (end 112.725 111.725) (width 0.2) (layer "F.Cu") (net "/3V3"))
 (segment (start 123.5 118) (end 126.725 118) (width 0.2) (layer "F.Cu") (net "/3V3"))
 (segment (start 121.1 114) (end 113 114) (width 0.2) (layer "F.Cu") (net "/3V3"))
 (segment (start 119.749911 116.5) (end 121.9 116.5) (width 0.2) (layer "F.Cu") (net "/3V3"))
 (segment (start 113 112) (end 113 114) (width 0.2) (layer "F.Cu") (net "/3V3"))
 (segment (start 113 114) (end 113 115) (width 0.2) (layer "F.Cu") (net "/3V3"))
 (segment (start 127.2 117.525) (end 126.725 118) (width 0.2) (layer "F.Cu") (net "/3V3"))
 (segment (start 121.9 116.5) (end 122 116.6) (width 0.2) (layer "F.Cu") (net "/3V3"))
 (segment (start 113.1 117) (end 115.449911 117) (width 0.2) (layer "F.Cu") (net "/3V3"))
 (segment (start 114.225 122) (end 113.099911 122) (width 0.2) (layer "F.Cu") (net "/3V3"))
 (segment (start 105.599911 115) (end 105.874911 115.275) (width 0.2) (layer "F.Cu") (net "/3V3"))
 (segment (start 105.099911 115) (end 113 115) (width 0.2) (layer "F.Cu") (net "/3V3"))
 (segment (start 122.1 116.6) (end 123.5 118) (width 0.2) (layer "F.Cu") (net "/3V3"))
 (segment (start 122 114.9) (end 121.1 114) (width 0.2) (layer "F.Cu") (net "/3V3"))
 (segment (start 113 116.9) (end 113.1 117) (width 0.2) (layer "F.Cu") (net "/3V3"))
 (segment (start 127.2 116) (end 127.2 117.525) (width 0.2) (layer "F.Cu") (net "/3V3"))
 (via (at 113 118.1) (size 0.6) (drill 0.3) (layers "F.Cu" "B.Cu") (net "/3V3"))
 (via (at 113 116.9) (size 0.6) (drill 0.3) (layers "F.Cu" "B.Cu") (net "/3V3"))
 (via (at 122 116.6) (size 0.6) (drill 0.3) (layers "F.Cu" "B.Cu") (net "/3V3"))
 (via (at 122 114.9) (size 0.6) (drill 0.3) (layers "F.Cu" "B.Cu") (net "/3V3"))
 (segment (start 113 116.9) (end 113 118.1) (width 0.2) (layer "B.Cu") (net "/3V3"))
 (segment (start 122 116.6) (end 122 114.9) (width 0.2) (layer "B.Cu") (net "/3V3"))
 (segment (start 115.775 123.225) (end 115.5 123.5) (width 0.2) (layer "F.Cu") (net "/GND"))
 (segment (start 114.275 108.049911) (end 114.324911 108) (width 0.2) (layer "F.Cu") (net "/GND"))
 (segment (start 115.599911 123.599911) (end 115.5 123.5) (width 0.2) (layer "F.Cu") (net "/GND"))
 (segment (start 114.324911 106) (end 114.324911 108) (width 0.2) (layer "F.Cu") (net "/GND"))
 (segment (start 114.275 111) (end 114.275 108.049911) (width 0.2) (layer "F.Cu") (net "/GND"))
 (segment (start 110.325 116.5) (end 111 116.5) (width 0.2) (layer "F.Cu") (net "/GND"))
 (segment (start 115.775 122) (end 115.775 123.225) (width 0.2) (layer "F.Cu") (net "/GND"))
 (segment (start 115.449911 115.5) (end 114.5 115.5) (width 0.2) (layer "F.Cu") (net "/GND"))
 (segment (start 111 116.5) (end 111.5 116) (width 0.2) (layer "F.Cu") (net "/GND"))
 (segment (start 114.5 116.5) (end 114 116) (width 0.2) (layer "F.Cu") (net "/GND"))
 (segment (start 122 119.275) (end 122 120.5) (width 0.2) (layer "F.Cu") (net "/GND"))
 (segment (start 128.275 118) (end 128.275 120.275) (width 0.2) (layer "F.Cu") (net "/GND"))
 (segment (start 119.5 121.275) (end 119.5 122.5) (width 0.2) (layer "F.Cu") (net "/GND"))
 (segment (start 105.2125 111) (end 103.5 111) (width 0.2) (layer "F.Cu") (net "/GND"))
 (segment (start 128 117.725) (end 128.275 118) (width 0.2) (layer "F.Cu") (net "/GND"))
 (segment (start 128 116) (end 128 117.725) (width 0.2) (layer "F.Cu") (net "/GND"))
 (segment (start 115.449911 116.5) (end 114.5 116.5) (width 0.2) (layer "F.Cu") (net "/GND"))
 (segment (start 114.5 115.5) (end 114 116) (width 0.2) (layer "F.Cu") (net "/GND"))
 (segment (start 115.599911 126.975) (end 115.599911 123.599911) (width 0.2) (layer "F.Cu") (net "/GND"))
 (segment (start 128.275 120.275) (end 128.5 120.5) (width 0.2) (layer "F.Cu") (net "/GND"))
 (via (at 115.5 123.5) (size 0.6) (drill 0.3) (layers "F.Cu" "B.Cu") (free yes) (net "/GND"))
 (via (at 103.5 111) (size 0.6) (drill 0.3) (layers "F.Cu" "B.Cu") (free yes) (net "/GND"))
 (via (at 114 116) (size 0.6) (drill 0.3) (layers "F.Cu" "B.Cu") (free yes) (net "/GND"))
 (via (at 122 120.5) (size 0.6) (drill 0.3) (layers "F.Cu" "B.Cu") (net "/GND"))
 (via (at 111.5 116) (size 0.6) (drill 0.3) (layers "F.Cu" "B.Cu") (free yes) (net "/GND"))
 (via (at 114.324911 108) (size 0.6) (drill 0.3) (layers "F.Cu" "B.Cu") (free yes) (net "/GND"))
 (via (at 128.5 120.5) (size 0.6) (drill 0.3) (layers "F.Cu" "B.Cu") (free yes) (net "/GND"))
 (via (at 119.5 122.5) (size 0.6) (drill 0.3) (layers "F.Cu" "B.Cu") (free yes) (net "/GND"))
 (segment (start 126.732843 114.032843) (end 127.2 114.5) (width 0.2) (layer "F.Cu") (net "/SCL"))
 (segment (start 116.824911 106) (end 116.824911 107.324911) (width 0.2) (layer "F.Cu") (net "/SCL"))
 (segment (start 116.824911 107.324911) (end 121.25 111.75) (width 0.2) (layer "F.Cu") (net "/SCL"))
 (segment (start 124.5 114.032843) (end 126.732843 114.032843) (width 0.2) (layer "F.Cu") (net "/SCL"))
 (segment (start 123.032843 115.5) (end 124.5 114.032843) (width 0.2) (layer "F.Cu") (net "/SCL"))
 (segment (start 123.532843 114.032843) (end 124.5 114.032843) (width 0.2) (layer "F.Cu") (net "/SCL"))
 (segment (start 121.25 111.75) (end 123.532843 114.032843) (width 0.2) (layer "F.Cu") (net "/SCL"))
 (segment (start 119.749911 115.5) (end 123.032843 115.5) (width 0.2) (layer "F.Cu") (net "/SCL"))
 (segment (start 127.2 114.5) (end 127.2 114.6) (width 0.2) (layer "F.Cu") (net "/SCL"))
 (segment (start 128 114.4) (end 127.1 113.5) (width 0.2) (layer "F.Cu") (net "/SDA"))
 (segment (start 125 113) (end 124.5 113.5) (width 0.2) (layer "F.Cu") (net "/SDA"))
 (segment (start 124.5 113.5) (end 123.565686 113.5) (width 0.2) (layer "F.Cu") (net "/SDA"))
 (segment (start 119 106) (end 119.324911 106) (width 0.2) (layer "F.Cu") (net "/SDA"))
 (segment (start 119.099911 106.165597) (end 119.099911 106) (width 0.2) (layer "F.Cu") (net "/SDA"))
 (segment (start 123.381373 116) (end 124.624265 114.757108) (width 0.2) (layer "F.Cu") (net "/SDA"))
 (segment (start 119.749911 116) (end 123.381373 116) (width 0.2) (layer "F.Cu") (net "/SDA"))
 (segment (start 121.532843 111.467157) (end 117.532843 107.467157) (width 0.2) (layer "F.Cu") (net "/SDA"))
 (segment (start 127.1 113.5) (end 124.5 113.5) (width 0.2) (layer "F.Cu") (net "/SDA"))
 (segment (start 128 114.6) (end 128 114.4) (width 0.2) (layer "F.Cu") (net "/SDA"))
 (segment (start 123.565686 113.5) (end 121.532843 111.467157) (width 0.2) (layer "F.Cu") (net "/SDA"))
 (segment (start 117.532843 107.467157) (end 119 106) (width 0.2) (layer "F.Cu") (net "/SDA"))
 (via (at 125 113) (size 0.6) (drill 0.3) (layers "F.Cu" "B.Cu") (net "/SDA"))
 (via (at 124.624265 114.757108) (size 0.6) (drill 0.3) (layers "F.Cu" "B.Cu") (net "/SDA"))
 (segment (start 124.624265 114.757108) (end 125 114.381373) (width 0.2) (layer "B.Cu") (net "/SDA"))
 (segment (start 125 114.381373) (end 125 113) (width 0.2) (layer "B.Cu") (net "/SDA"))
 (segment (start 108.675 117.325) (end 108.5 117.5) (width 0.2) (layer "F.Cu") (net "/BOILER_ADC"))
 (segment (start 108.675 116.5) (end 108.675 117.325) (width 0.2) (layer "F.Cu") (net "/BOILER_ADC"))
 (segment (start 108.7375 116.5) (end 109 116.7625) (width 0.2) (layer "F.Cu") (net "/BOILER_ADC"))
 (segment (start 115.449911 117.5) (end 108.5 117.5) (width 0.2) (layer "F.Cu") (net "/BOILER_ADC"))
 (segment (start 108.5 117.5) (end 105.099911 117.5) (width 0.2) (layer "F.Cu") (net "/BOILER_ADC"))
 (segment (start 108.675 111) (end 106.7875 111) (width 0.2) (layer "F.Cu") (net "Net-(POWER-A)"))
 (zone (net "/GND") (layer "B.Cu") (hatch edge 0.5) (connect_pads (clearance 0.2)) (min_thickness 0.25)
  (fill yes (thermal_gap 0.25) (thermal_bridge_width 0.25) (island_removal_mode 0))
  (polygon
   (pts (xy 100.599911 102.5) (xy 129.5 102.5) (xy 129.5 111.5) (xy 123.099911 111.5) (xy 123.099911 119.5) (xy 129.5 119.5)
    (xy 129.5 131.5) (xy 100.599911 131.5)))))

